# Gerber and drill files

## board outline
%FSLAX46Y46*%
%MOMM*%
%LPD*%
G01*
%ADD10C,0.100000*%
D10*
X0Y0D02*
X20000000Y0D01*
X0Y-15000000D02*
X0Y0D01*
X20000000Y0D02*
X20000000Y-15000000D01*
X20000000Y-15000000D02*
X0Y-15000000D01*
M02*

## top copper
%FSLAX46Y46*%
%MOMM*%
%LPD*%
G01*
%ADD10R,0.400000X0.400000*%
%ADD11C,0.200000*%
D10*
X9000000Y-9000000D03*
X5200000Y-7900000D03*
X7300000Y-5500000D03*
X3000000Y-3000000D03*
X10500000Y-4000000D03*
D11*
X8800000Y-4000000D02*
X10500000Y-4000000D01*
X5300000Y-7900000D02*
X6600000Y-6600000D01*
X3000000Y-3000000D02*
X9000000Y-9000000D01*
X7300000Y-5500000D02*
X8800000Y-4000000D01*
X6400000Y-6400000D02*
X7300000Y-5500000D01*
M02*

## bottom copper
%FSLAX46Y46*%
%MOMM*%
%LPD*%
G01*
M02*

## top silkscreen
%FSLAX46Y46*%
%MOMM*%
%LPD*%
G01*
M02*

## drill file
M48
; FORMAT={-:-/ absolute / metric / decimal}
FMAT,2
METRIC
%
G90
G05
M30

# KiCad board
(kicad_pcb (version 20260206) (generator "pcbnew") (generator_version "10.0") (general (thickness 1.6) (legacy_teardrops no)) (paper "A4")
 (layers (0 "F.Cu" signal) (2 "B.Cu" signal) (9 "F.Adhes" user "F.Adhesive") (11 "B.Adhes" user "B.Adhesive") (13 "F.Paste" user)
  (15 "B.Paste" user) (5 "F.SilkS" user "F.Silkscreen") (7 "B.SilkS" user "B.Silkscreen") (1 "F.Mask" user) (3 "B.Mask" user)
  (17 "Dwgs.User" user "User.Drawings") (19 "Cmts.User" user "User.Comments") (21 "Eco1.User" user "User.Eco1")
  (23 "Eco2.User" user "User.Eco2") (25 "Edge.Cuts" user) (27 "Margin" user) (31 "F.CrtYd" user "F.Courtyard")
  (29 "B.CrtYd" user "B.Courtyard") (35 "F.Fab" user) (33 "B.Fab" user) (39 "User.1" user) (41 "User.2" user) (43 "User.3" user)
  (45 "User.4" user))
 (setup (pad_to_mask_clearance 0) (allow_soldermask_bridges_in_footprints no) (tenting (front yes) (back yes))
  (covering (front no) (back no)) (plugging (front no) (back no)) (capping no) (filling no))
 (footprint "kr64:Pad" (layer "F.Cu") (at 9 9)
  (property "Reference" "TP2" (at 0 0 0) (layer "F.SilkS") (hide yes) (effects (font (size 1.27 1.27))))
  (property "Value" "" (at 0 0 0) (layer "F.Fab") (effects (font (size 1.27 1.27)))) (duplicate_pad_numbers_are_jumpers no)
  (pad "1" smd rect (at 0 0) (size 0.4 0.4) (layers "F.Cu" "F.Mask" "F.Paste") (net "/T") (thermal_bridge_angle 45)))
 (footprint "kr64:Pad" (layer "F.Cu") (at 5.2 7.9)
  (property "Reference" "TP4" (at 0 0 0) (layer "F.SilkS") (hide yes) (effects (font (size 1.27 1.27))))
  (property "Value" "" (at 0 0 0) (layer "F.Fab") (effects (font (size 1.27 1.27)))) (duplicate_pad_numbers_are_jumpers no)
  (pad "1" smd rect (at 0 0) (size 0.4 0.4) (layers "F.Cu" "F.Mask" "F.Paste") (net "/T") (thermal_bridge_angle 45)))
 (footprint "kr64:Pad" (layer "F.Cu") (at 7.3 5.5)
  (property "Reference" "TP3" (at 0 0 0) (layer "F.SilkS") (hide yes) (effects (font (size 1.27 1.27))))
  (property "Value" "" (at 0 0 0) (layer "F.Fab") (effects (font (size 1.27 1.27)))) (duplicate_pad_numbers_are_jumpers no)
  (pad "1" smd rect (at 0 0) (size 0.4 0.4) (layers "F.Cu" "F.Mask" "F.Paste") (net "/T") (thermal_bridge_angle 45)))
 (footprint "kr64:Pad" (layer "F.Cu") (at 3 3)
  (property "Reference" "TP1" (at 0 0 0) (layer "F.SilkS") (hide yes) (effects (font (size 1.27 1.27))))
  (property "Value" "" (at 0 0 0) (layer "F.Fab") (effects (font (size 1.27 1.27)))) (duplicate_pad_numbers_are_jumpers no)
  (pad "1" smd rect (at 0 0) (size 0.4 0.4) (layers "F.Cu" "F.Mask" "F.Paste") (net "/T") (thermal_bridge_angle 45)))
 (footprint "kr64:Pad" (layer "F.Cu") (at 10.5 4)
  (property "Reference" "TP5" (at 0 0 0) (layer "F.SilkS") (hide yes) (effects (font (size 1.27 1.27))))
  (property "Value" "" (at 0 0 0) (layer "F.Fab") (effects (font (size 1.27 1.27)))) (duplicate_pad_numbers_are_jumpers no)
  (pad "1" smd rect (at 0 0) (size 0.4 0.4) (layers "F.Cu" "F.Mask" "F.Paste") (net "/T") (thermal_bridge_angle 45)))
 (gr_line (start 0 0) (end 20 0) (stroke (width 0.1) (type default)) (layer "Edge.Cuts"))
 (gr_line (start 0 15) (end 0 0) (stroke (width 0.1) (type default)) (layer "Edge.Cuts"))
 (gr_line (start 20 0) (end 20 15) (stroke (width 0.1) (type default)) (layer "Edge.Cuts"))
 (gr_line (start 20 15) (end 0 15) (stroke (width 0.1) (type default)) (layer "Edge.Cuts"))
 (segment (start 8.8 4) (end 10.5 4) (width 0.2) (layer "F.Cu") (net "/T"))
 (segment (start 5.3 7.9) (end 6.6 6.6) (width 0.2) (layer "F.Cu") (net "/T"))
 (segment (start 3 3) (end 9 9) (width 0.2) (layer "F.Cu") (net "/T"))
 (segment (start 7.3 5.5) (end 8.8 4) (width 0.2) (layer "F.Cu") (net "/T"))
 (segment (start 6.4 6.4) (end 7.3 5.5) (width 0.2) (layer "F.Cu") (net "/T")))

